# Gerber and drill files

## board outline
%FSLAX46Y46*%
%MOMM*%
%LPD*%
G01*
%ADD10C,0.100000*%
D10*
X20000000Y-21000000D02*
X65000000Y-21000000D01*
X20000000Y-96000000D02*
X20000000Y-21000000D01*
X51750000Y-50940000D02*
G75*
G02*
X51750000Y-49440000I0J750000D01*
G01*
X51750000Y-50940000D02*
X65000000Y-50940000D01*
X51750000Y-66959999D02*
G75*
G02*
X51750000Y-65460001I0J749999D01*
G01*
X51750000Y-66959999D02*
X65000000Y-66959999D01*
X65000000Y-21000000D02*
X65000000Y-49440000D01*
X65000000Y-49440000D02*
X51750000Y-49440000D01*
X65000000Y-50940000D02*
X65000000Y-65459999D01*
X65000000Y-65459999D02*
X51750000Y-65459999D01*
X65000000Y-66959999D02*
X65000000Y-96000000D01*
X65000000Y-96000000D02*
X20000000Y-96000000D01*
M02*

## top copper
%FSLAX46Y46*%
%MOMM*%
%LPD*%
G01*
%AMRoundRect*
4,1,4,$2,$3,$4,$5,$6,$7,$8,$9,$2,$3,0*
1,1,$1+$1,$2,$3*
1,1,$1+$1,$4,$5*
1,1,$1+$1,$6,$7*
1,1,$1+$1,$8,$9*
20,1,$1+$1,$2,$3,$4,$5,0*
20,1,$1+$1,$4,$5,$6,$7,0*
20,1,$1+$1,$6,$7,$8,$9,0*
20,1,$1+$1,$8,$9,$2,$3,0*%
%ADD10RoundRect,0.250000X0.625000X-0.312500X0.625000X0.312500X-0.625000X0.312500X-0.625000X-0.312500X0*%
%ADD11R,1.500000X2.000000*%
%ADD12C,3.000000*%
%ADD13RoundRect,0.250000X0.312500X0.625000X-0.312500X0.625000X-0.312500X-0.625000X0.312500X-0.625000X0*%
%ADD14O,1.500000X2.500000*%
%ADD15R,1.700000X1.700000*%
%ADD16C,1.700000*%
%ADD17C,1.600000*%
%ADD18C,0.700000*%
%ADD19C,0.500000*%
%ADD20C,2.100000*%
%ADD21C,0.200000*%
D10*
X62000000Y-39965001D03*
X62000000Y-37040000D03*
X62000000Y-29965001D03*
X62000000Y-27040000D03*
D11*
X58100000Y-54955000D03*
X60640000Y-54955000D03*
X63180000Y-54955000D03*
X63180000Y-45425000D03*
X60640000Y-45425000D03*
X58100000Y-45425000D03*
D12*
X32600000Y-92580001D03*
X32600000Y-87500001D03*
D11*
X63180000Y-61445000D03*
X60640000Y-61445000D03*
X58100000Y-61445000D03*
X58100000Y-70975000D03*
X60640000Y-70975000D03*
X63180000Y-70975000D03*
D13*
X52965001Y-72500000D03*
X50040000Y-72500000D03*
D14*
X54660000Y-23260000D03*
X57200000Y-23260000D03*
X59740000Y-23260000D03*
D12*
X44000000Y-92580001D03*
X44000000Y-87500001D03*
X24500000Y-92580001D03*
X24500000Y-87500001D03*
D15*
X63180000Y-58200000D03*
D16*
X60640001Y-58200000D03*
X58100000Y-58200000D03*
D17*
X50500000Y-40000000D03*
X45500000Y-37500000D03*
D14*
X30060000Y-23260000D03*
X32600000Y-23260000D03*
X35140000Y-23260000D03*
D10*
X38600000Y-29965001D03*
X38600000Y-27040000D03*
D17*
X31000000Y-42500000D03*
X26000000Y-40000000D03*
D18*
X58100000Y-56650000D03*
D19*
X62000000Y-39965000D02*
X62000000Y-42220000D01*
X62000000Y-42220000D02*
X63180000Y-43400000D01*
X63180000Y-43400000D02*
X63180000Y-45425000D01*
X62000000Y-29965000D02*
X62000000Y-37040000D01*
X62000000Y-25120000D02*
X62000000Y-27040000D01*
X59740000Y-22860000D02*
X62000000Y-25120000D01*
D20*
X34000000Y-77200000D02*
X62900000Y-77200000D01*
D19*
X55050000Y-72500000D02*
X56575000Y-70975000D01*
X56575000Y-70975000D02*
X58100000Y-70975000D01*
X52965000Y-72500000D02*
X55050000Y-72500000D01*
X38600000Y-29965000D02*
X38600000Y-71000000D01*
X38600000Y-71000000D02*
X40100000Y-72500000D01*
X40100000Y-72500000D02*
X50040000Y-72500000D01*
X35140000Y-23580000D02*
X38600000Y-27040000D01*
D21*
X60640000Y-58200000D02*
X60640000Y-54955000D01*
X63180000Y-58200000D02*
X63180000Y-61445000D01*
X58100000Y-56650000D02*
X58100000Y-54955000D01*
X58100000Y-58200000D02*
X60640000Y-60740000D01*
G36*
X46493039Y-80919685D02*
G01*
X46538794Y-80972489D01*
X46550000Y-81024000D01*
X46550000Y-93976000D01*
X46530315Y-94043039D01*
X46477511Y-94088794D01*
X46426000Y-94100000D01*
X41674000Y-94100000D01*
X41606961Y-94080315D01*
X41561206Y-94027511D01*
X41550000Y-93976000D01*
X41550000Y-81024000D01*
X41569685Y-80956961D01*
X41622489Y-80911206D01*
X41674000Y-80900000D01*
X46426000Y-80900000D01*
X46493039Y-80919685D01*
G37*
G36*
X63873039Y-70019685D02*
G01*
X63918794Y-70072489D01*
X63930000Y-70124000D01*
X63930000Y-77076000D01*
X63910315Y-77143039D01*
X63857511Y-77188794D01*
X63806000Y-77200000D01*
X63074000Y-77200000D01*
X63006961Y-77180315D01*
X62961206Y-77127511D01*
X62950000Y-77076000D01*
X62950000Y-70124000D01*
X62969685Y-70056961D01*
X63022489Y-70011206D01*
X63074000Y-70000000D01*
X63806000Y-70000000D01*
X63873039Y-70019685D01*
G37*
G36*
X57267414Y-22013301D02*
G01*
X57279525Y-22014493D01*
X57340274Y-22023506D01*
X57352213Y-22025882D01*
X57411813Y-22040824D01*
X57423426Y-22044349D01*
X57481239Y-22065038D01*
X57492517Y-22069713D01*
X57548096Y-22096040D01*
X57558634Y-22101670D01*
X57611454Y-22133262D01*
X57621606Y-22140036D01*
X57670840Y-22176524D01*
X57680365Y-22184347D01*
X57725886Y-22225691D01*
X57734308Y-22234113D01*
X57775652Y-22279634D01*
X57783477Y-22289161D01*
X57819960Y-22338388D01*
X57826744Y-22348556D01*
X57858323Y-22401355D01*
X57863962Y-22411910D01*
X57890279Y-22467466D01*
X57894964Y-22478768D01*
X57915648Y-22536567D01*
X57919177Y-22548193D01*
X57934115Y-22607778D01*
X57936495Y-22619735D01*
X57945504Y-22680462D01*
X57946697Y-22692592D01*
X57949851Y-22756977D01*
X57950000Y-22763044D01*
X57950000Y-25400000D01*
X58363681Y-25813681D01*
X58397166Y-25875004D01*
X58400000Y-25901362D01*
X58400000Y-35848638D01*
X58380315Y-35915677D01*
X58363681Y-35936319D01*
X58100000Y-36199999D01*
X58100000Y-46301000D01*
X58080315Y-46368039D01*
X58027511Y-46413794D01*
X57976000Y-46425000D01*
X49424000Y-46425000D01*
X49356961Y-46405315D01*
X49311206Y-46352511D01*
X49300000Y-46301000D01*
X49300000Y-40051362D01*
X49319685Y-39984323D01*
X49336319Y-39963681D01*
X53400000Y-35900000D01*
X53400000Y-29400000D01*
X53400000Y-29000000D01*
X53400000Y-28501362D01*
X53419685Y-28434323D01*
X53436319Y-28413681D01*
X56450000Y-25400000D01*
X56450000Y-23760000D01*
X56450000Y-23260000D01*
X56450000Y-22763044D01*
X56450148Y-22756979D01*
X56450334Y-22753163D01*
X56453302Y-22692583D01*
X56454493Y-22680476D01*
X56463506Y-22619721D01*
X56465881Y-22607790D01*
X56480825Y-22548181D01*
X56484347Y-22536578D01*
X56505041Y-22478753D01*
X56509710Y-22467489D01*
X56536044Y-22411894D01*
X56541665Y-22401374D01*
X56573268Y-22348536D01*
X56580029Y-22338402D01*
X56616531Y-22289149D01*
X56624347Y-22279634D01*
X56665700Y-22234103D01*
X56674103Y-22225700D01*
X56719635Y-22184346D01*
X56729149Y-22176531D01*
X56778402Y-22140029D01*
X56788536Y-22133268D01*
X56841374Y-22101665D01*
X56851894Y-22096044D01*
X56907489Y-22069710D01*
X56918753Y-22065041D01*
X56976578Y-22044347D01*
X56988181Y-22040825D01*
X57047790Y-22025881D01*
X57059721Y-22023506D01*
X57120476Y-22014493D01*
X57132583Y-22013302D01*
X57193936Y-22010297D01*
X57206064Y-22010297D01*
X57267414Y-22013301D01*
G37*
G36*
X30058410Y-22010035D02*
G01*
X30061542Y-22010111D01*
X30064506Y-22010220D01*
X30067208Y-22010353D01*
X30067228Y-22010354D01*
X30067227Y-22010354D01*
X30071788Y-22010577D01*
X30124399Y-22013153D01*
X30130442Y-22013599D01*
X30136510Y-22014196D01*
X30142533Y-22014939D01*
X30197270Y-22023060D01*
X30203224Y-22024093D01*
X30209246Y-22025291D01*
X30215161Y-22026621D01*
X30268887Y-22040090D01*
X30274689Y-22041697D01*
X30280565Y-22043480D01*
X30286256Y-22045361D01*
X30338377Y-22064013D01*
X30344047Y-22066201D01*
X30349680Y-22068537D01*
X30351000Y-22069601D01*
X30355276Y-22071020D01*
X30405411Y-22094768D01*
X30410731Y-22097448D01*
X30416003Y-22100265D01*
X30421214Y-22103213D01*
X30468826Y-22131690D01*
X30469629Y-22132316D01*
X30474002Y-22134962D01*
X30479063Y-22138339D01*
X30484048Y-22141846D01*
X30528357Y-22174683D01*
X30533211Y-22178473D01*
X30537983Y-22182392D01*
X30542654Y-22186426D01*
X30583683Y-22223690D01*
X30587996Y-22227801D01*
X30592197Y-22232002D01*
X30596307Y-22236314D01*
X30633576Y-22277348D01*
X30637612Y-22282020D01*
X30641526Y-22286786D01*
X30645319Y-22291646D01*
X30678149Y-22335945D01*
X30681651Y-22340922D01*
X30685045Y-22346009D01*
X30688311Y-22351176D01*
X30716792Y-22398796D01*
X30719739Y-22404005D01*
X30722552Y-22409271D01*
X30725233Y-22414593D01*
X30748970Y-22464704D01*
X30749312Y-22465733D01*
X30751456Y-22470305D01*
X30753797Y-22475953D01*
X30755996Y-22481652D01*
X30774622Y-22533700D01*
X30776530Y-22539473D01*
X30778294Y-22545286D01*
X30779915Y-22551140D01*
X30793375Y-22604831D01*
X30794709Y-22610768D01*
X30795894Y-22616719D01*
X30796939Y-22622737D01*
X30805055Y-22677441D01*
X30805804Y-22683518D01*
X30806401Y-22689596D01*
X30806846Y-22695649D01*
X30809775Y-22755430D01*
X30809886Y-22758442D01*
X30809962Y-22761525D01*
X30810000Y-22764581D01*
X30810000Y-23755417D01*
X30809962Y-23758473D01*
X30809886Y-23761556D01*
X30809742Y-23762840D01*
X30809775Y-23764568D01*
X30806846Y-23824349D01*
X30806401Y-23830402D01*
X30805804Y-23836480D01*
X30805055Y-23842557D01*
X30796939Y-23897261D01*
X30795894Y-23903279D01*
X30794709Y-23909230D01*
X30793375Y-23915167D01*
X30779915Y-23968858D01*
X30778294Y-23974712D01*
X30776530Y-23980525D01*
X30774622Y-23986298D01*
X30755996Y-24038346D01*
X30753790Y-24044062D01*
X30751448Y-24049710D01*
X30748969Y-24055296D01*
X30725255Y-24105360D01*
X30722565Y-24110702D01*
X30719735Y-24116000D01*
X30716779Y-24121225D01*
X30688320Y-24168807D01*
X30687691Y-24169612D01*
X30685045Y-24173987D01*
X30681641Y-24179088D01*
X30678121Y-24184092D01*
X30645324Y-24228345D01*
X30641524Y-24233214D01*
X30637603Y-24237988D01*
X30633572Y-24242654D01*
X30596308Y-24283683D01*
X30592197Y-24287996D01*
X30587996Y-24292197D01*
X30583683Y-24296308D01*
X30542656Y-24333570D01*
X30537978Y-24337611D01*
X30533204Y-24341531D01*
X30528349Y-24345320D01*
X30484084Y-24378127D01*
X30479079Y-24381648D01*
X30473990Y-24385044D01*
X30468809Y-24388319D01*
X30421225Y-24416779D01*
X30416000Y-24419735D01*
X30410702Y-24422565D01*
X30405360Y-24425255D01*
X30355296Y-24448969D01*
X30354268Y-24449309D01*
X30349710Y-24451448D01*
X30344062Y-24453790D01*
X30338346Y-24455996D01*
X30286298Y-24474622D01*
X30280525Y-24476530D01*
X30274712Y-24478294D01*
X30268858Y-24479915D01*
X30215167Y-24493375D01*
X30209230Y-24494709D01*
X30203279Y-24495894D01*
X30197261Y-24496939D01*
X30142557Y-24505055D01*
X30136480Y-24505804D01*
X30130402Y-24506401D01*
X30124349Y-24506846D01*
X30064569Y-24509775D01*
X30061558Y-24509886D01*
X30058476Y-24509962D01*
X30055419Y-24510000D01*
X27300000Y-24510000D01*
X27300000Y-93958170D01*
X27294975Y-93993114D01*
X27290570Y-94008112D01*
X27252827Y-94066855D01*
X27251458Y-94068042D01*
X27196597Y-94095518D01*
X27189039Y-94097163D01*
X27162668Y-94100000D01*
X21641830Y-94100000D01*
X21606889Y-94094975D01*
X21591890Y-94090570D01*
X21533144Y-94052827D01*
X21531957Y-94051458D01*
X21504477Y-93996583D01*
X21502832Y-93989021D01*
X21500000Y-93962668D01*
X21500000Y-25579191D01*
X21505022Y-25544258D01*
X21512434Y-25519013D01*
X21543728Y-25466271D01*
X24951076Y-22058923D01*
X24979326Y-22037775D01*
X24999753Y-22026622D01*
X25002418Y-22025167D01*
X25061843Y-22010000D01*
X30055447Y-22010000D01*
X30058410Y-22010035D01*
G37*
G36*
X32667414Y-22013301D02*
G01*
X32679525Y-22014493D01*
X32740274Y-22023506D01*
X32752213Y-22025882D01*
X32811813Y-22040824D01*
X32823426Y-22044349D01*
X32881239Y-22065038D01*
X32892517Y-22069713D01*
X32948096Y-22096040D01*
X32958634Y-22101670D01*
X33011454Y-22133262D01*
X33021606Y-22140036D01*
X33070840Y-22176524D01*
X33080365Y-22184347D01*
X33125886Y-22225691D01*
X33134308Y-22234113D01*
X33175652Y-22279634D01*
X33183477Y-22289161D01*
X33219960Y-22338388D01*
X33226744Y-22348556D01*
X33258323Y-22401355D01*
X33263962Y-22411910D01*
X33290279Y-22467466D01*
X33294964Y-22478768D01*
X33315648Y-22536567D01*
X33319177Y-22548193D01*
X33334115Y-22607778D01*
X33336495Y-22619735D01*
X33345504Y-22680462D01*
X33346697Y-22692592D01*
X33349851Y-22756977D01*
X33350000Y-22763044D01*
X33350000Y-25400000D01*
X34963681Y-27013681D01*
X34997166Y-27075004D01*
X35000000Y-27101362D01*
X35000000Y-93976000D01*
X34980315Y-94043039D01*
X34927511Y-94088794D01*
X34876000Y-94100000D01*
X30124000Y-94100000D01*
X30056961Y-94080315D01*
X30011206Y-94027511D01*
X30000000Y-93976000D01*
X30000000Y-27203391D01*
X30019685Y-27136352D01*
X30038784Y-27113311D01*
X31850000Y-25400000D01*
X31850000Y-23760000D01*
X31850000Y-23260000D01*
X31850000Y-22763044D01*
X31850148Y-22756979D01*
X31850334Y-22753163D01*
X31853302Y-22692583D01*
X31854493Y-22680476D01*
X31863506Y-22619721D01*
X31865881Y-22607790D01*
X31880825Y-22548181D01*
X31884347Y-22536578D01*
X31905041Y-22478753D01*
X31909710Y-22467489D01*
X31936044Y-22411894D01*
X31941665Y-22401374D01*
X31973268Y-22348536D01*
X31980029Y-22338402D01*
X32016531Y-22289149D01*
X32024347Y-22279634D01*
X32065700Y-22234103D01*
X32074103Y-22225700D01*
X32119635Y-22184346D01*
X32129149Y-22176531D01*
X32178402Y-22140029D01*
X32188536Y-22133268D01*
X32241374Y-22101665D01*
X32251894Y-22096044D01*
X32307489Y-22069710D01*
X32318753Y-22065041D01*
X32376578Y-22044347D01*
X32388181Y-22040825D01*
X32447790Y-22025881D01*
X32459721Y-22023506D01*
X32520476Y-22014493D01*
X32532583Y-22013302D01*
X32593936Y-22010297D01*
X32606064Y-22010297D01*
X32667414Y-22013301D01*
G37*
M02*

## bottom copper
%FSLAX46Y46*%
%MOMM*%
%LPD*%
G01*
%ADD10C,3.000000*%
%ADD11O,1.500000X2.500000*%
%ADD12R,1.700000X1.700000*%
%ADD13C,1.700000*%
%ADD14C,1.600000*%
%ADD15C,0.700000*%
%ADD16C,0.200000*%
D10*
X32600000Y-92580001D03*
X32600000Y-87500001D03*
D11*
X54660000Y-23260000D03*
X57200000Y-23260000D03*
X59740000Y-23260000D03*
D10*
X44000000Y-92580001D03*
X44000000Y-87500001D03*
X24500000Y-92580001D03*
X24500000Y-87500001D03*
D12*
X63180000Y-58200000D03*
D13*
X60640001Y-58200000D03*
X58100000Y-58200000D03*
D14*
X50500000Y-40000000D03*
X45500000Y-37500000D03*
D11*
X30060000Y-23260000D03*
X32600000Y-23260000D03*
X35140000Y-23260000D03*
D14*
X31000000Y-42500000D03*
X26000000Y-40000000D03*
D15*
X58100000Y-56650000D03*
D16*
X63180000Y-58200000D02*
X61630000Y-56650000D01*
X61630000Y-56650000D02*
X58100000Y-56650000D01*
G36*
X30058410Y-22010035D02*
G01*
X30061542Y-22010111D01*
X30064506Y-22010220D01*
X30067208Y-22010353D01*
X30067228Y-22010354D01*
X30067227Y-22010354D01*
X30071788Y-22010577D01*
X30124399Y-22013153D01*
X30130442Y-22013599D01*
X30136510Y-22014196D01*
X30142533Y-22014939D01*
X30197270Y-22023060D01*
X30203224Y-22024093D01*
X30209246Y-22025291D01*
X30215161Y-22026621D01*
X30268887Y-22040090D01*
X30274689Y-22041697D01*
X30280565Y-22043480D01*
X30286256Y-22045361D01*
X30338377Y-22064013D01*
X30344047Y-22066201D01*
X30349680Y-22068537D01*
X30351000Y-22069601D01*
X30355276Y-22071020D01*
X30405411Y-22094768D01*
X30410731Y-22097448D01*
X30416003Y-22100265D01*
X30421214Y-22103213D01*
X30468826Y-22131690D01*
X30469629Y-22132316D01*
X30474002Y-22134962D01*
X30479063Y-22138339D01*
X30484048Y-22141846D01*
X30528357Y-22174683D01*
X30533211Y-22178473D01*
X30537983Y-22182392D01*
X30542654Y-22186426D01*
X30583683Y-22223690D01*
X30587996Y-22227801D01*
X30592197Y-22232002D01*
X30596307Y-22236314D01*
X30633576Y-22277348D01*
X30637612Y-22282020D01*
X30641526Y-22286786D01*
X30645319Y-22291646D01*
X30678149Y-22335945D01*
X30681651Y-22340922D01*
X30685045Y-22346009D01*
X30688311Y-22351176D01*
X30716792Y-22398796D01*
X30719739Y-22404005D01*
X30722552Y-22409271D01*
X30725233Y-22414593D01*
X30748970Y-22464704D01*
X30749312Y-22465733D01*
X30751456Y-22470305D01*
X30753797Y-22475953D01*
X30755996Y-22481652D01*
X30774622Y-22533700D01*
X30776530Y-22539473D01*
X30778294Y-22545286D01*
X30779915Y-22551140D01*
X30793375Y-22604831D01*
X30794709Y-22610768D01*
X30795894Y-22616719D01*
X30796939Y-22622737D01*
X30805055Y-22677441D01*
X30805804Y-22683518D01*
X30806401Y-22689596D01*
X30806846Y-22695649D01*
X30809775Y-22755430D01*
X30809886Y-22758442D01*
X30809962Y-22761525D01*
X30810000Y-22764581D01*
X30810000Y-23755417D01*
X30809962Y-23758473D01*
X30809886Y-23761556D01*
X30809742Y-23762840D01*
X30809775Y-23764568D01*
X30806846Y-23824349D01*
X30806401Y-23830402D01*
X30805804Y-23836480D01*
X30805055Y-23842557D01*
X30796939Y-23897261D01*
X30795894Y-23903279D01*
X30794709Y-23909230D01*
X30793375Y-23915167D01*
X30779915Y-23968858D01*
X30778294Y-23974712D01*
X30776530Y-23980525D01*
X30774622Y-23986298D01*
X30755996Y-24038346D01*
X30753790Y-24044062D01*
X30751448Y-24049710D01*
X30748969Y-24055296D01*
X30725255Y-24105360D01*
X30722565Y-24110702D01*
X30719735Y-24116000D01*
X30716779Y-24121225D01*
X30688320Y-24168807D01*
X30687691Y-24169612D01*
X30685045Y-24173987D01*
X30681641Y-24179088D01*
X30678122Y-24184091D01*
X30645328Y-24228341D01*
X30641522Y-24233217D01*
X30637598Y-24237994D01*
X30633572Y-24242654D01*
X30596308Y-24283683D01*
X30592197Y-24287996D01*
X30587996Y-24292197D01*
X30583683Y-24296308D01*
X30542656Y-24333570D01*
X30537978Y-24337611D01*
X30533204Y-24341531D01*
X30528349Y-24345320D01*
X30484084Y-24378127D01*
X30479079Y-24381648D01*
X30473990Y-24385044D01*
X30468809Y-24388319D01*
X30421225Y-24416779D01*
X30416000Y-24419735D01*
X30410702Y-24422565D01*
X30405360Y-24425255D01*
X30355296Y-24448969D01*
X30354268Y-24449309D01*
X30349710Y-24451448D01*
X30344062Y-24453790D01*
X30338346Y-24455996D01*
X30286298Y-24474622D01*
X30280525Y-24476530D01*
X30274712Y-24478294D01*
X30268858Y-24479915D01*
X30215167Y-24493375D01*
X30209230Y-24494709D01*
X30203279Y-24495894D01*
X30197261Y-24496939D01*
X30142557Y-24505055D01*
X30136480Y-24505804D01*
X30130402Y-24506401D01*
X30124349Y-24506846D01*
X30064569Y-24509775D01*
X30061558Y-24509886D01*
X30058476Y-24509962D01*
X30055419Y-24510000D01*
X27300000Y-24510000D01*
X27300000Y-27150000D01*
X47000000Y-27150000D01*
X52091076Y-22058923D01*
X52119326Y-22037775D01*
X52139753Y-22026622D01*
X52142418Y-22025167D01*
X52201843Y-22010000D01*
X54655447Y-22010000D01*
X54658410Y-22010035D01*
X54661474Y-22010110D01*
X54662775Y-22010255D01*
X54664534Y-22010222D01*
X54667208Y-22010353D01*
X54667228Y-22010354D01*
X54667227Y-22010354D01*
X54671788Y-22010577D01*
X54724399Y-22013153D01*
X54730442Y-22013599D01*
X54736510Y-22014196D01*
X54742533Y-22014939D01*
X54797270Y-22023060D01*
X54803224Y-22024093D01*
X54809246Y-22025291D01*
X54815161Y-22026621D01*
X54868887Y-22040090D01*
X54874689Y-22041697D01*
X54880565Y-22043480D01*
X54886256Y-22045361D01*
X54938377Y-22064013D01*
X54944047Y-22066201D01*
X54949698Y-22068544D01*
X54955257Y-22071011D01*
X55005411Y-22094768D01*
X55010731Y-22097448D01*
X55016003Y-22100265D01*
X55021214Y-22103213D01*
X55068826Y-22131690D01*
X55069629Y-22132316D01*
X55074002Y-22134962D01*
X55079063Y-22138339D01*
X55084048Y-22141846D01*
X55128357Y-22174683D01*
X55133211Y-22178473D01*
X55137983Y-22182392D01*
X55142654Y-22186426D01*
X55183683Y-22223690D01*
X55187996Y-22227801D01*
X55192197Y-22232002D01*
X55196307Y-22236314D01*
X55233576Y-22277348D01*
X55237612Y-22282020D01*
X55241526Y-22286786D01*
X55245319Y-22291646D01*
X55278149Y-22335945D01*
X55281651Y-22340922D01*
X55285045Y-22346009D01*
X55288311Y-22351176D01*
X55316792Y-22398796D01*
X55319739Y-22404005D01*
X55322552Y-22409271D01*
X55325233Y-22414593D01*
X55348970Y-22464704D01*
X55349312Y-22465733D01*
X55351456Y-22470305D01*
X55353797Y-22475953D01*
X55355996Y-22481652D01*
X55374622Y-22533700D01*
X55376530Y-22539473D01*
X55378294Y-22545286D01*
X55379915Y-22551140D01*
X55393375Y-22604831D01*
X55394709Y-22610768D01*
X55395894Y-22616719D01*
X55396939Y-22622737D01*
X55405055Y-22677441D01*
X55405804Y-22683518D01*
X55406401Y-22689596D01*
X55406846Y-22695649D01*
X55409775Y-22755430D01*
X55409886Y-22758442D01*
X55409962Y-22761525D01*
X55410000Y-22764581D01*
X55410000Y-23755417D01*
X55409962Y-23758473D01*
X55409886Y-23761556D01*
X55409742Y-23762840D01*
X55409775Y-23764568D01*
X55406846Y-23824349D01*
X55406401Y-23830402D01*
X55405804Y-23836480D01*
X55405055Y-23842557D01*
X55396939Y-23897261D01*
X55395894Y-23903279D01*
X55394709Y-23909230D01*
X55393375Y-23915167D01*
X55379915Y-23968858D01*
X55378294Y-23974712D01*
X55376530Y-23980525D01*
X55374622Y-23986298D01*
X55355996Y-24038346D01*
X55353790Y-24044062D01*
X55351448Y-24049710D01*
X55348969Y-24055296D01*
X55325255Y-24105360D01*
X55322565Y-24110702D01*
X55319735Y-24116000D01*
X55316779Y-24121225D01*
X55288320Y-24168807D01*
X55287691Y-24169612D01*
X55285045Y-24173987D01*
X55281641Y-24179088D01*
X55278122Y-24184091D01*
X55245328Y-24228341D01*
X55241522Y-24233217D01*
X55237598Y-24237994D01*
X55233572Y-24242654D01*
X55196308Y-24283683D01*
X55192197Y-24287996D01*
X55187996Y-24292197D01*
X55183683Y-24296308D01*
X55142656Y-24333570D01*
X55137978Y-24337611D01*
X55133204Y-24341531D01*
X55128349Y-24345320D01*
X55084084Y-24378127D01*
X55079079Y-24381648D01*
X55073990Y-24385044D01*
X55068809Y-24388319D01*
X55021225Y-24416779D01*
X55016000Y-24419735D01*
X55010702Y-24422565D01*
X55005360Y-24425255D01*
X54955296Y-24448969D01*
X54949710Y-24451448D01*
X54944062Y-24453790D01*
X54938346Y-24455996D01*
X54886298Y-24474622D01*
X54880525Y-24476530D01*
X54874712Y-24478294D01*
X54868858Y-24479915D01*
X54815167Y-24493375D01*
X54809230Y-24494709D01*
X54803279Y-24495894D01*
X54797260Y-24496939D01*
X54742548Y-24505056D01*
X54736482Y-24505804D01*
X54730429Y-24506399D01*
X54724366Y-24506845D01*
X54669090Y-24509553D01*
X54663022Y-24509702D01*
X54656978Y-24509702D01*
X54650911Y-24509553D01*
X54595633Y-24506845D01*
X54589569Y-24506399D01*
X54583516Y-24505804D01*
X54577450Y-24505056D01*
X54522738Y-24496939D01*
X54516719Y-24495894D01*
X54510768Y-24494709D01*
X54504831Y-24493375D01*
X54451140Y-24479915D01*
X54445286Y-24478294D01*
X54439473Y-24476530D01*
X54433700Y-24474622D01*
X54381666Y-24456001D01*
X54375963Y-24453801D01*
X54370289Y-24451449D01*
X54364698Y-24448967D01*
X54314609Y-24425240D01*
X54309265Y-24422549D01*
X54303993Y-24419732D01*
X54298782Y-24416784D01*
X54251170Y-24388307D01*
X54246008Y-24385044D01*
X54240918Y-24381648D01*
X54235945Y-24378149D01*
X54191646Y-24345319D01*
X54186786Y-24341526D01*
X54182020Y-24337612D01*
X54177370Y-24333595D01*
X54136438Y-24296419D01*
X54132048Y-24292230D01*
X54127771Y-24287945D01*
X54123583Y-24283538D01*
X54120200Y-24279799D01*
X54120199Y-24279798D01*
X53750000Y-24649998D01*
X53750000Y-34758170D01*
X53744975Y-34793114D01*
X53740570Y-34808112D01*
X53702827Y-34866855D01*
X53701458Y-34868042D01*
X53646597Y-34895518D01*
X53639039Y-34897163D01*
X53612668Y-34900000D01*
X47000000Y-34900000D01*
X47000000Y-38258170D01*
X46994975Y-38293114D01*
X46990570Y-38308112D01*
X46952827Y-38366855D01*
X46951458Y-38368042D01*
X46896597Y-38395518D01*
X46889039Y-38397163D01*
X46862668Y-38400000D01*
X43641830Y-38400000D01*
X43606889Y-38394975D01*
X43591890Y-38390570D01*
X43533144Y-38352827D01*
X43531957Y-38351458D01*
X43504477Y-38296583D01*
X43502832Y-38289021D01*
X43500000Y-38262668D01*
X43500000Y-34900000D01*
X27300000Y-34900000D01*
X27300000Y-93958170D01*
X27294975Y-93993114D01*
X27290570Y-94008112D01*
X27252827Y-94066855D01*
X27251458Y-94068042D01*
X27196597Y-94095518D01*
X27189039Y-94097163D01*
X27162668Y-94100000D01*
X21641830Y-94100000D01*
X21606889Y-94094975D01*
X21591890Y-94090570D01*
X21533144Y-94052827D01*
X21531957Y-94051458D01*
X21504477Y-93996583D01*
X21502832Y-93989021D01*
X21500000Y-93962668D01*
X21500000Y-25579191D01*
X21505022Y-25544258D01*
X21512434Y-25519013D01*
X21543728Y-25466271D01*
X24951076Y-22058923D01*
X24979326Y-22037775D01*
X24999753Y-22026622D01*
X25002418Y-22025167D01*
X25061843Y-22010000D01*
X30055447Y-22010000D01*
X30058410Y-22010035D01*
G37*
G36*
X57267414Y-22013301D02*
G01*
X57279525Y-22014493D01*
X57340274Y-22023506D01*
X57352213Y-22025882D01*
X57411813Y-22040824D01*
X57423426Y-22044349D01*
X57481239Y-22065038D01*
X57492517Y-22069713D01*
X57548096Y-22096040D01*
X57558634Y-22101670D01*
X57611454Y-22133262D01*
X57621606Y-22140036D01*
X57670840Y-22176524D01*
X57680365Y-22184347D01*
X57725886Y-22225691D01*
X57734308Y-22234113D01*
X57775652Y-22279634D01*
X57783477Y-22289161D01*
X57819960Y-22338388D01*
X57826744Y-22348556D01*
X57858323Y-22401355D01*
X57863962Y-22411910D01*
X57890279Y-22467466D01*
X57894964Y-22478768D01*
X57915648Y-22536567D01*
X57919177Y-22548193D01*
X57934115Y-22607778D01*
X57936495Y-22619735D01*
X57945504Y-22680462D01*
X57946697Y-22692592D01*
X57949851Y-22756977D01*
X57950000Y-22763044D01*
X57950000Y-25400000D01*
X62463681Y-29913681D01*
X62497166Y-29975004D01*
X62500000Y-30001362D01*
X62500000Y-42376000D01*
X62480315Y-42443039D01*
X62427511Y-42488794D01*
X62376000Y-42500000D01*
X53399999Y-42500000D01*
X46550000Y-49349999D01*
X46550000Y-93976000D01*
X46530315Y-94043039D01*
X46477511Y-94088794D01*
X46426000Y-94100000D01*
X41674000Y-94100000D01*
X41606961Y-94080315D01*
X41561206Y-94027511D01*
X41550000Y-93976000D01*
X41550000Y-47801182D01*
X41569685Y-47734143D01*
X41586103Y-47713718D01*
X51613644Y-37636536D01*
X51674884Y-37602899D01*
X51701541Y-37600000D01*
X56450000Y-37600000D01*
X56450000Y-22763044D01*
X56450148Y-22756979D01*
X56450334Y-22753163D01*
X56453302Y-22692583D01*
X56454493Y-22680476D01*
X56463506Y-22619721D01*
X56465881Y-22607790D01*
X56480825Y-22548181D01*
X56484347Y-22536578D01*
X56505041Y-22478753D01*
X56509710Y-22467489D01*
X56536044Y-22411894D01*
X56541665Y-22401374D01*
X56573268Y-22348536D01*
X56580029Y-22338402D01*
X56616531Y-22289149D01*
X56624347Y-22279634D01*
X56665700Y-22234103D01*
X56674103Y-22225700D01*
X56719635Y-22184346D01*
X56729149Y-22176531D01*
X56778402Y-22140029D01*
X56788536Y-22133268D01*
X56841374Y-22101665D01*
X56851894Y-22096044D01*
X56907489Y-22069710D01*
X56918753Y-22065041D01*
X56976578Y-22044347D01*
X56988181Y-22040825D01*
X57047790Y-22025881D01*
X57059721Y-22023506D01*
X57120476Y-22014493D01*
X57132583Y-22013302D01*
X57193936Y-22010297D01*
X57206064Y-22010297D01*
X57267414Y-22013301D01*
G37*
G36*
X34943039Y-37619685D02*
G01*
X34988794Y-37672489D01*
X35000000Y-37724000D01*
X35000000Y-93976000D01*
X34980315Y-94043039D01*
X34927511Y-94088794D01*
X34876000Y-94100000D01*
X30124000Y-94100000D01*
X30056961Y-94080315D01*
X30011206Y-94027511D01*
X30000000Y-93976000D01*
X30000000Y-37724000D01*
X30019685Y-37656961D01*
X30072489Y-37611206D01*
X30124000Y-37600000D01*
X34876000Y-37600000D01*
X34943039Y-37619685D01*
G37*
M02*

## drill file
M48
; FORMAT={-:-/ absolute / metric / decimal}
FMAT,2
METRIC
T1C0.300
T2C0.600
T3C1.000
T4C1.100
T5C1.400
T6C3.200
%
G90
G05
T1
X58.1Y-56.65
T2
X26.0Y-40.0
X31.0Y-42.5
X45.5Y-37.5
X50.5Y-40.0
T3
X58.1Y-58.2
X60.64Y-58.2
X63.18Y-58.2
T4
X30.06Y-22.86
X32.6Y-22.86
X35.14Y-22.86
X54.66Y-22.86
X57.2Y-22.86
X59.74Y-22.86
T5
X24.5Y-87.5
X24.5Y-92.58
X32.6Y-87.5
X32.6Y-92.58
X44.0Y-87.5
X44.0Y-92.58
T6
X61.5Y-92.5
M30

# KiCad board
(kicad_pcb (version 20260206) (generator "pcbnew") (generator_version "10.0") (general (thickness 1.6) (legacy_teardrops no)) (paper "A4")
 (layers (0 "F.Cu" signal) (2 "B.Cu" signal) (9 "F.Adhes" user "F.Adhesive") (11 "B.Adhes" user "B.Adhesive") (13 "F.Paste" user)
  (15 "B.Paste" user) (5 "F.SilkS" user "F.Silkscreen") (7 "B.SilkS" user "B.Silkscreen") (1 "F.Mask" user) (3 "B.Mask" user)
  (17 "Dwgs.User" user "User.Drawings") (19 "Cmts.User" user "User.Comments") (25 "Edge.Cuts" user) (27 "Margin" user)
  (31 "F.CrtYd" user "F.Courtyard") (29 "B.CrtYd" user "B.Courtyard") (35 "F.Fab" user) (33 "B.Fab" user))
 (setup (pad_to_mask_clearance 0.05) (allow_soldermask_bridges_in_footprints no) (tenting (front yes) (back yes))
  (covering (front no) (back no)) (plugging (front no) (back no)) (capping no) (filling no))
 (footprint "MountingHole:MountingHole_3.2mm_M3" (layer "F.Cu") (at 61.5 92.5)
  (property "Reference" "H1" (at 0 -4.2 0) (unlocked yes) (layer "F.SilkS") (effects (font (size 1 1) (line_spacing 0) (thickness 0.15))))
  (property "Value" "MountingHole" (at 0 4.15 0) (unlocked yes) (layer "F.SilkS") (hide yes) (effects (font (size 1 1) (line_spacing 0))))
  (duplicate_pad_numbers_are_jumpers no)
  (pad "" np_thru_hole circle (at 0 0) (size 3.2 3.2) (drill 3.2) (layers "*.Cu" "*.Mask")))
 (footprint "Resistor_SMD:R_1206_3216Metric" (layer "F.Cu") (at 62 38.502501 90)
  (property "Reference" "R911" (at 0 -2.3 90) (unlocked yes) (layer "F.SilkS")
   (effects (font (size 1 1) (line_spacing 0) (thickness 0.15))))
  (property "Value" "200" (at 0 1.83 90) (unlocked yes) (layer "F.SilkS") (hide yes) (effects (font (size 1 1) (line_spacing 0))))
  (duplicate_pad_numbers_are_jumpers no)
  (pad "1" smd roundrect (at -1.4625 0 90) (size 1.125 1.75) (layers "F.Cu" "F.Mask" "F.Paste") (roundrect_rratio 0.222222)
   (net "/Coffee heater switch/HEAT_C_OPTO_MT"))
  (pad "2" smd roundrect (at 1.462501 0 90) (size 1.125 1.75) (layers "F.Cu" "F.Mask" "F.Paste") (roundrect_rratio 0.222222)
   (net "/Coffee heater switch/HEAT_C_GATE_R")))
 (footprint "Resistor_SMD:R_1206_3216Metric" (layer "F.Cu") (at 62 28.502501 90)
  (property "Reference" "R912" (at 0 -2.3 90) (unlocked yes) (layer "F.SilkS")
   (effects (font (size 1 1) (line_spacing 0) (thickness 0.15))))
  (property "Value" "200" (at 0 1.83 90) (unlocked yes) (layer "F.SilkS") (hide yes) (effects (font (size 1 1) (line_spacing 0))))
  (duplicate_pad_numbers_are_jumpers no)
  (pad "1" smd roundrect (at -1.4625 0 90) (size 1.125 1.75) (layers "F.Cu" "F.Mask" "F.Paste") (roundrect_rratio 0.222222)
   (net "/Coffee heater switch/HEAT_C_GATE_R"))
  (pad "2" smd roundrect (at 1.462501 0 90) (size 1.125 1.75) (layers "F.Cu" "F.Mask" "F.Paste") (roundrect_rratio 0.222222)
   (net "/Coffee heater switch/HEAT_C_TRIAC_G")))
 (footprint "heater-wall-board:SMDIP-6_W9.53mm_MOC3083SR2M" (layer "F.Cu") (at 60.64 50.19 90)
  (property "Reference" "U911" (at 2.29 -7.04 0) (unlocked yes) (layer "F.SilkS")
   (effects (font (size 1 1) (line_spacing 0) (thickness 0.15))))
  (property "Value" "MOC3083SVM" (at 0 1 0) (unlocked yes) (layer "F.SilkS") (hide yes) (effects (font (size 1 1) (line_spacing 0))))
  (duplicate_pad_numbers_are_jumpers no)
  (pad "1" smd rect (at -4.765 -2.54 90) (size 2 1.5) (layers "F.Cu" "F.Mask" "F.Paste") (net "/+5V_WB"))
  (pad "2" smd rect (at -4.765 0 90) (size 2 1.5) (layers "F.Cu" "F.Mask" "F.Paste") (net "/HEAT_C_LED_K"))
  (pad "3" smd rect (at -4.765 2.54 90) (size 2 1.5) (layers "F.Cu" "F.Mask" "F.Paste") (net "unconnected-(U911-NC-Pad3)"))
  (pad "4" smd rect (at 4.765 2.54 90) (size 2 1.5) (layers "F.Cu" "F.Mask" "F.Paste") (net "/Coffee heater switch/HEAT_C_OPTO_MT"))
  (pad "5" smd rect (at 4.765 0 90) (size 2 1.5) (layers "F.Cu" "F.Mask" "F.Paste") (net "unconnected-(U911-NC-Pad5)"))
  (pad "6" smd rect (at 4.765 -2.54 90) (size 2 1.5) (layers "F.Cu" "F.Mask" "F.Paste") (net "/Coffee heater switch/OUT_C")))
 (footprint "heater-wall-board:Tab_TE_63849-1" (layer "F.Cu") (at 32.6 90.04 90)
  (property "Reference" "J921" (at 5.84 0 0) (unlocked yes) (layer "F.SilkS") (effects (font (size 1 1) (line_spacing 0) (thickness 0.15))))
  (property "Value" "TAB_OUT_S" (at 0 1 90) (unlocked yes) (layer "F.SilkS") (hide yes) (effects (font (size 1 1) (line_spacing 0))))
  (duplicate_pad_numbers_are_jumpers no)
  (pad "1" thru_hole circle (at -2.540001 0 90) (size 3 3) (drill 1.4) (layers "*.Cu" "*.Mask") (remove_unused_layers no)
   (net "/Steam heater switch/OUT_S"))
  (pad "1" thru_hole circle (at 2.539999 0 90) (size 3 3) (drill 1.4) (layers "*.Cu" "*.Mask") (remove_unused_layers no)
   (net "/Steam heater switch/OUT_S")))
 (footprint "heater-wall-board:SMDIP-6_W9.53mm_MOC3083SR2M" (layer "F.Cu") (at 60.64 66.21 -90)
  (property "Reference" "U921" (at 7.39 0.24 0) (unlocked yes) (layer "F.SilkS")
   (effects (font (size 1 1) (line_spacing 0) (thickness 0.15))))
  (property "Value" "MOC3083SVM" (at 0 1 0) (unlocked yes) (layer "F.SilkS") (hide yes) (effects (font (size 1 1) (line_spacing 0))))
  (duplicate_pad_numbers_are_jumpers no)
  (pad "1" smd rect (at -4.765 -2.54 270) (size 2 1.5) (layers "F.Cu" "F.Mask" "F.Paste") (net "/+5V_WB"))
  (pad "2" smd rect (at -4.765 0 270) (size 2 1.5) (layers "F.Cu" "F.Mask" "F.Paste") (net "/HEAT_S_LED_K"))
  (pad "3" smd rect (at -4.765 2.54 270) (size 2 1.5) (layers "F.Cu" "F.Mask" "F.Paste") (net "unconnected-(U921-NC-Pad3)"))
  (pad "4" smd rect (at 4.765 2.54 270) (size 2 1.5) (layers "F.Cu" "F.Mask" "F.Paste") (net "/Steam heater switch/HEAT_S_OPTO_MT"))
  (pad "5" smd rect (at 4.765 0 270) (size 2 1.5) (layers "F.Cu" "F.Mask" "F.Paste") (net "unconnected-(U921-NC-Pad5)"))
  (pad "6" smd rect (at 4.765 -2.54 270) (size 2 1.5) (layers "F.Cu" "F.Mask" "F.Paste") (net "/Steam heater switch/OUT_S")))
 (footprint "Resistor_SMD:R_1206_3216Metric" (layer "F.Cu") (at 51.502501 72.5 180)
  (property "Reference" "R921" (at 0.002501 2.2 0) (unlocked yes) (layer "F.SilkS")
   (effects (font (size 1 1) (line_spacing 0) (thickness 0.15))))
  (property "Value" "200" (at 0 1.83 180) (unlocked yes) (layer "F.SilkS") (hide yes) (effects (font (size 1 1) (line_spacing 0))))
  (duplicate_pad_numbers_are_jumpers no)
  (pad "1" smd roundrect (at -1.4625 0 180) (size 1.125 1.75) (layers "F.Cu" "F.Mask" "F.Paste") (roundrect_rratio 0.222222)
   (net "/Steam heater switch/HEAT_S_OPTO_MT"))
  (pad "2" smd roundrect (at 1.462501 0 180) (size 1.125 1.75) (layers "F.Cu" "F.Mask" "F.Paste") (roundrect_rratio 0.222222)
   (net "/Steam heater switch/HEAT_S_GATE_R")))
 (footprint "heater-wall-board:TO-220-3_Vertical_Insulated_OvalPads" (layer "F.Cu") (at 54.66 22.86)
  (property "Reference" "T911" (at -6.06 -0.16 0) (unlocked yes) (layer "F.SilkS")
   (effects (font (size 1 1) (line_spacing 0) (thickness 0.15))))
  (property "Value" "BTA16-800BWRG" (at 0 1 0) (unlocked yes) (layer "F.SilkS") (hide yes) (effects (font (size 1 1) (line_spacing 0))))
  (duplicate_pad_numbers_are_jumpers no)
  (pad "1" thru_hole oval (at 0 0) (size 1.5 2.5) (drill 1.1 (offset 0 0.4)) (layers "*.Cu" "*.Mask") (remove_unused_layers no) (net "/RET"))
  (pad "2" thru_hole oval (at 2.54 0) (size 1.5 2.5) (drill 1.1 (offset 0 0.4)) (layers "*.Cu" "*.Mask") (remove_unused_layers no)
   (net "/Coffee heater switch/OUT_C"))
  (pad "3" thru_hole oval (at 5.08 0) (size 1.5 2.5) (drill 1.1 (offset 0 0.4)) (layers "*.Cu" "*.Mask") (remove_unused_layers no)
   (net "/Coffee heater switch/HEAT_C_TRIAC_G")))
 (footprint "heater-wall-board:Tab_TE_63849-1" (layer "F.Cu") (at 44 90.04 90)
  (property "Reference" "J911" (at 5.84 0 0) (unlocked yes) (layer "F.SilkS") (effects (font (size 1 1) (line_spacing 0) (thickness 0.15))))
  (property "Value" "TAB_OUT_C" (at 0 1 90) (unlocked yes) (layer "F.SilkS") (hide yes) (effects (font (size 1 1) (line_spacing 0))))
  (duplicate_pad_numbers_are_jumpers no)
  (pad "1" thru_hole circle (at -2.540001 0 90) (size 3 3) (drill 1.4) (layers "*.Cu" "*.Mask") (remove_unused_layers no)
   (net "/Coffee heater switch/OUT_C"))
  (pad "1" thru_hole circle (at 2.539999 0 90) (size 3 3) (drill 1.4) (layers "*.Cu" "*.Mask") (remove_unused_layers no)
   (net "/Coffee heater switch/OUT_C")))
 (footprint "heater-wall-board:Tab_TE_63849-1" (layer "F.Cu") (at 24.5 90.04 90)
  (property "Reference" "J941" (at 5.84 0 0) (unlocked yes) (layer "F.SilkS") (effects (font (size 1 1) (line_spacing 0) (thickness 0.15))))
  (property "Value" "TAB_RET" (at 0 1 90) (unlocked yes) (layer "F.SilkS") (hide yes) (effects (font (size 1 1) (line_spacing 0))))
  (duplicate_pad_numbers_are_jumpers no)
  (pad "1" thru_hole circle (at -2.540001 0 90) (size 3 3) (drill 1.4) (layers "*.Cu" "*.Mask") (remove_unused_layers no) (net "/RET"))
  (pad "1" thru_hole circle (at 2.539999 0 90) (size 3 3) (drill 1.4) (layers "*.Cu" "*.Mask") (remove_unused_layers no) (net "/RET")))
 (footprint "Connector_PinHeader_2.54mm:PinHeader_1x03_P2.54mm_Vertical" (layer "F.Cu") (at 63.18 58.2 -90)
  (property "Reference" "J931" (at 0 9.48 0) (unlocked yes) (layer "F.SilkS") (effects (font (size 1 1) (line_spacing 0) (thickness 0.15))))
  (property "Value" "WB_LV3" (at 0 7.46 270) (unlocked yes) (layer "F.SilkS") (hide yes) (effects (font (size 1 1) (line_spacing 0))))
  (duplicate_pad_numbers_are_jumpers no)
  (pad "1" thru_hole rect (at 0 0 270) (size 1.7 1.7) (drill 1) (layers "*.Cu" "*.Mask") (remove_unused_layers no) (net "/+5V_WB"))
  (pad "2" thru_hole circle (at 0 2.539999 270) (size 1.7 1.7) (drill 1) (layers "*.Cu" "*.Mask") (remove_unused_layers no)
   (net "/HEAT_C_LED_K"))
  (pad "3" thru_hole circle (at 0 5.08 270) (size 1.7 1.7) (drill 1) (layers "*.Cu" "*.Mask") (remove_unused_layers no)
   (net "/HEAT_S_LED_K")))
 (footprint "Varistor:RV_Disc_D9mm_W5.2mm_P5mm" (layer "F.Cu") (at 50.5 40 180)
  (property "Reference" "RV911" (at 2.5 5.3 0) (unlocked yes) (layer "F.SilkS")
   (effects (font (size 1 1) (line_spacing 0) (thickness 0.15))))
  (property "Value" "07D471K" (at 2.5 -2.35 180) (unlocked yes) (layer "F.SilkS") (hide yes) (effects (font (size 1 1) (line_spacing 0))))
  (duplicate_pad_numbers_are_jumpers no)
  (pad "1" thru_hole circle (at 0 0 180) (size 1.6 1.6) (drill 0.6) (layers "*.Cu" "*.Mask") (remove_unused_layers no)
   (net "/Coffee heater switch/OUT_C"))
  (pad "2" thru_hole circle (at 5 2.5 180) (size 1.6 1.6) (drill 0.6) (layers "*.Cu" "*.Mask") (remove_unused_layers no) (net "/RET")))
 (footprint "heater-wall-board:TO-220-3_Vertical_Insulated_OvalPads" (layer "F.Cu") (at 30.06 22.86)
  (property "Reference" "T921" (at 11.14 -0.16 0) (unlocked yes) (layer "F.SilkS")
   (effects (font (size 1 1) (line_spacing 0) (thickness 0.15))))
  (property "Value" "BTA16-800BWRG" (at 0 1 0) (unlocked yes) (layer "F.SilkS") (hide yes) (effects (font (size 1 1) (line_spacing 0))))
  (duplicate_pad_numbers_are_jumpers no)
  (pad "1" thru_hole oval (at 0 0) (size 1.5 2.5) (drill 1.1 (offset 0 0.4)) (layers "*.Cu" "*.Mask") (remove_unused_layers no) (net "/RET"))
  (pad "2" thru_hole oval (at 2.54 0) (size 1.5 2.5) (drill 1.1 (offset 0 0.4)) (layers "*.Cu" "*.Mask") (remove_unused_layers no)
   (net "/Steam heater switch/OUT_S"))
  (pad "3" thru_hole oval (at 5.08 0) (size 1.5 2.5) (drill 1.1 (offset 0 0.4)) (layers "*.Cu" "*.Mask") (remove_unused_layers no)
   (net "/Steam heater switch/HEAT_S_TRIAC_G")))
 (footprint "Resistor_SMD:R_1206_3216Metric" (layer "F.Cu") (at 38.6 28.502501 90)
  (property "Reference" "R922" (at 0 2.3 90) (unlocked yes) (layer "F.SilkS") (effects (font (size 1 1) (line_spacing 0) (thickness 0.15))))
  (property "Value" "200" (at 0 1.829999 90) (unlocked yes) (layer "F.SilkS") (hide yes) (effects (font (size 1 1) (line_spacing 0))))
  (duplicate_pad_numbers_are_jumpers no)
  (pad "1" smd roundrect (at -1.4625 0 90) (size 1.125 1.75) (layers "F.Cu" "F.Mask" "F.Paste") (roundrect_rratio 0.222222)
   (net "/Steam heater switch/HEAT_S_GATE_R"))
  (pad "2" smd roundrect (at 1.462501 0 90) (size 1.125 1.75) (layers "F.Cu" "F.Mask" "F.Paste") (roundrect_rratio 0.222222)
   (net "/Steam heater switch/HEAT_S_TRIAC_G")))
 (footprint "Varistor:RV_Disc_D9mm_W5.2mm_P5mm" (layer "F.Cu") (at 31 42.5 180)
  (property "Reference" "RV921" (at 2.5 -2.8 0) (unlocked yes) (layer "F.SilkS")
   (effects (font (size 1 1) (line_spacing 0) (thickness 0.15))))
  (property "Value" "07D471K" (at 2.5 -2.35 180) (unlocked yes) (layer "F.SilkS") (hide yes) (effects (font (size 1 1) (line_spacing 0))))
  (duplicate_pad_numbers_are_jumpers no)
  (pad "1" thru_hole circle (at 0 0 180) (size 1.6 1.6) (drill 0.6) (layers "*.Cu" "*.Mask") (remove_unused_layers no)
   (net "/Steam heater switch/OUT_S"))
  (pad "2" thru_hole circle (at 5 2.5 180) (size 1.6 1.6) (drill 0.6) (layers "*.Cu" "*.Mask") (remove_unused_layers no) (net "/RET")))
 (gr_line (start 20 21) (end 65 21) (stroke (width 0.1) (type default)) (layer "Edge.Cuts"))
 (gr_line (start 20 96) (end 20 21) (stroke (width 0.1) (type default)) (layer "Edge.Cuts"))
 (gr_arc (start 51.75 50.94) (mid 51 50.19) (end 51.75 49.44) (stroke (width 0.1) (type default)) (layer "Edge.Cuts"))
 (gr_line (start 51.75 50.94) (end 65 50.94) (stroke (width 0.1) (type default)) (layer "Edge.Cuts"))
 (gr_arc (start 51.75 66.959999) (mid 51.000001 66.21) (end 51.75 65.459999) (stroke (width 0.1) (type default)) (layer "Edge.Cuts"))
 (gr_line (start 51.75 66.959999) (end 65 66.959999) (stroke (width 0.1) (type default)) (layer "Edge.Cuts"))
 (gr_line (start 65 21) (end 65 49.44) (stroke (width 0.1) (type default)) (layer "Edge.Cuts"))
 (gr_line (start 65 49.44) (end 51.75 49.44) (stroke (width 0.1) (type default)) (layer "Edge.Cuts"))
 (gr_line (start 65 50.94) (end 65 65.459999) (stroke (width 0.1) (type default)) (layer "Edge.Cuts"))
 (gr_line (start 65 65.459999) (end 51.75 65.459999) (stroke (width 0.1) (type default)) (layer "Edge.Cuts"))
 (gr_line (start 65 66.959999) (end 65 96) (stroke (width 0.1) (type default)) (layer "Edge.Cuts"))
 (gr_line (start 65 96) (end 20 96) (stroke (width 0.1) (type default)) (layer "Edge.Cuts"))
 (segment (start 62 39.965) (end 62 42.22) (width 0.5) (locked yes) (layer "F.Cu") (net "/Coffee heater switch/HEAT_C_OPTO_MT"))
 (segment (start 62 42.22) (end 63.18 43.4) (width 0.5) (locked yes) (layer "F.Cu") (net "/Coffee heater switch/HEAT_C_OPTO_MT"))
 (segment (start 63.18 43.4) (end 63.18 45.425) (width 0.5) (locked yes) (layer "F.Cu") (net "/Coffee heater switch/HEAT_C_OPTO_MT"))
 (segment (start 62 29.965) (end 62 37.04) (width 0.5) (locked yes) (layer "F.Cu") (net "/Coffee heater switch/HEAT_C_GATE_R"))
 (segment (start 62 25.12) (end 62 27.04) (width 0.5) (locked yes) (layer "F.Cu") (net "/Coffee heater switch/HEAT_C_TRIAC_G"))
 (segment (start 59.74 22.86) (end 62 25.12) (width 0.5) (locked yes) (layer "F.Cu") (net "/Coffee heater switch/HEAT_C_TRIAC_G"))
 (segment (start 34 77.2) (end 62.9 77.2) (width 2.1) (locked yes) (layer "F.Cu") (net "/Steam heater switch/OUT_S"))
 (segment (start 55.05 72.5) (end 56.575 70.975) (width 0.5) (locked yes) (layer "F.Cu") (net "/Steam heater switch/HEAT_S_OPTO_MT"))
 (segment (start 56.575 70.975) (end 58.1 70.975) (width 0.5) (locked yes) (layer "F.Cu") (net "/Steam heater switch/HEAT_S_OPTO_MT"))
 (segment (start 52.965 72.5) (end 55.05 72.5) (width 0.5) (locked yes) (layer "F.Cu") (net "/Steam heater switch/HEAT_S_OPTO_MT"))
 (segment (start 38.6 29.965) (end 38.6 71) (width 0.5) (locked yes) (layer "F.Cu") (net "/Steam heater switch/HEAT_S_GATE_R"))
 (segment (start 38.6 71) (end 40.1 72.5) (width 0.5) (locked yes) (layer "F.Cu") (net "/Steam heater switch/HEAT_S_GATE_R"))
 (segment (start 40.1 72.5) (end 50.04 72.5) (width 0.5) (locked yes) (layer "F.Cu") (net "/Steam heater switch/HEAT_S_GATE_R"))
 (segment (start 35.14 23.58) (end 38.6 27.04) (width 0.5) (locked yes) (layer "F.Cu") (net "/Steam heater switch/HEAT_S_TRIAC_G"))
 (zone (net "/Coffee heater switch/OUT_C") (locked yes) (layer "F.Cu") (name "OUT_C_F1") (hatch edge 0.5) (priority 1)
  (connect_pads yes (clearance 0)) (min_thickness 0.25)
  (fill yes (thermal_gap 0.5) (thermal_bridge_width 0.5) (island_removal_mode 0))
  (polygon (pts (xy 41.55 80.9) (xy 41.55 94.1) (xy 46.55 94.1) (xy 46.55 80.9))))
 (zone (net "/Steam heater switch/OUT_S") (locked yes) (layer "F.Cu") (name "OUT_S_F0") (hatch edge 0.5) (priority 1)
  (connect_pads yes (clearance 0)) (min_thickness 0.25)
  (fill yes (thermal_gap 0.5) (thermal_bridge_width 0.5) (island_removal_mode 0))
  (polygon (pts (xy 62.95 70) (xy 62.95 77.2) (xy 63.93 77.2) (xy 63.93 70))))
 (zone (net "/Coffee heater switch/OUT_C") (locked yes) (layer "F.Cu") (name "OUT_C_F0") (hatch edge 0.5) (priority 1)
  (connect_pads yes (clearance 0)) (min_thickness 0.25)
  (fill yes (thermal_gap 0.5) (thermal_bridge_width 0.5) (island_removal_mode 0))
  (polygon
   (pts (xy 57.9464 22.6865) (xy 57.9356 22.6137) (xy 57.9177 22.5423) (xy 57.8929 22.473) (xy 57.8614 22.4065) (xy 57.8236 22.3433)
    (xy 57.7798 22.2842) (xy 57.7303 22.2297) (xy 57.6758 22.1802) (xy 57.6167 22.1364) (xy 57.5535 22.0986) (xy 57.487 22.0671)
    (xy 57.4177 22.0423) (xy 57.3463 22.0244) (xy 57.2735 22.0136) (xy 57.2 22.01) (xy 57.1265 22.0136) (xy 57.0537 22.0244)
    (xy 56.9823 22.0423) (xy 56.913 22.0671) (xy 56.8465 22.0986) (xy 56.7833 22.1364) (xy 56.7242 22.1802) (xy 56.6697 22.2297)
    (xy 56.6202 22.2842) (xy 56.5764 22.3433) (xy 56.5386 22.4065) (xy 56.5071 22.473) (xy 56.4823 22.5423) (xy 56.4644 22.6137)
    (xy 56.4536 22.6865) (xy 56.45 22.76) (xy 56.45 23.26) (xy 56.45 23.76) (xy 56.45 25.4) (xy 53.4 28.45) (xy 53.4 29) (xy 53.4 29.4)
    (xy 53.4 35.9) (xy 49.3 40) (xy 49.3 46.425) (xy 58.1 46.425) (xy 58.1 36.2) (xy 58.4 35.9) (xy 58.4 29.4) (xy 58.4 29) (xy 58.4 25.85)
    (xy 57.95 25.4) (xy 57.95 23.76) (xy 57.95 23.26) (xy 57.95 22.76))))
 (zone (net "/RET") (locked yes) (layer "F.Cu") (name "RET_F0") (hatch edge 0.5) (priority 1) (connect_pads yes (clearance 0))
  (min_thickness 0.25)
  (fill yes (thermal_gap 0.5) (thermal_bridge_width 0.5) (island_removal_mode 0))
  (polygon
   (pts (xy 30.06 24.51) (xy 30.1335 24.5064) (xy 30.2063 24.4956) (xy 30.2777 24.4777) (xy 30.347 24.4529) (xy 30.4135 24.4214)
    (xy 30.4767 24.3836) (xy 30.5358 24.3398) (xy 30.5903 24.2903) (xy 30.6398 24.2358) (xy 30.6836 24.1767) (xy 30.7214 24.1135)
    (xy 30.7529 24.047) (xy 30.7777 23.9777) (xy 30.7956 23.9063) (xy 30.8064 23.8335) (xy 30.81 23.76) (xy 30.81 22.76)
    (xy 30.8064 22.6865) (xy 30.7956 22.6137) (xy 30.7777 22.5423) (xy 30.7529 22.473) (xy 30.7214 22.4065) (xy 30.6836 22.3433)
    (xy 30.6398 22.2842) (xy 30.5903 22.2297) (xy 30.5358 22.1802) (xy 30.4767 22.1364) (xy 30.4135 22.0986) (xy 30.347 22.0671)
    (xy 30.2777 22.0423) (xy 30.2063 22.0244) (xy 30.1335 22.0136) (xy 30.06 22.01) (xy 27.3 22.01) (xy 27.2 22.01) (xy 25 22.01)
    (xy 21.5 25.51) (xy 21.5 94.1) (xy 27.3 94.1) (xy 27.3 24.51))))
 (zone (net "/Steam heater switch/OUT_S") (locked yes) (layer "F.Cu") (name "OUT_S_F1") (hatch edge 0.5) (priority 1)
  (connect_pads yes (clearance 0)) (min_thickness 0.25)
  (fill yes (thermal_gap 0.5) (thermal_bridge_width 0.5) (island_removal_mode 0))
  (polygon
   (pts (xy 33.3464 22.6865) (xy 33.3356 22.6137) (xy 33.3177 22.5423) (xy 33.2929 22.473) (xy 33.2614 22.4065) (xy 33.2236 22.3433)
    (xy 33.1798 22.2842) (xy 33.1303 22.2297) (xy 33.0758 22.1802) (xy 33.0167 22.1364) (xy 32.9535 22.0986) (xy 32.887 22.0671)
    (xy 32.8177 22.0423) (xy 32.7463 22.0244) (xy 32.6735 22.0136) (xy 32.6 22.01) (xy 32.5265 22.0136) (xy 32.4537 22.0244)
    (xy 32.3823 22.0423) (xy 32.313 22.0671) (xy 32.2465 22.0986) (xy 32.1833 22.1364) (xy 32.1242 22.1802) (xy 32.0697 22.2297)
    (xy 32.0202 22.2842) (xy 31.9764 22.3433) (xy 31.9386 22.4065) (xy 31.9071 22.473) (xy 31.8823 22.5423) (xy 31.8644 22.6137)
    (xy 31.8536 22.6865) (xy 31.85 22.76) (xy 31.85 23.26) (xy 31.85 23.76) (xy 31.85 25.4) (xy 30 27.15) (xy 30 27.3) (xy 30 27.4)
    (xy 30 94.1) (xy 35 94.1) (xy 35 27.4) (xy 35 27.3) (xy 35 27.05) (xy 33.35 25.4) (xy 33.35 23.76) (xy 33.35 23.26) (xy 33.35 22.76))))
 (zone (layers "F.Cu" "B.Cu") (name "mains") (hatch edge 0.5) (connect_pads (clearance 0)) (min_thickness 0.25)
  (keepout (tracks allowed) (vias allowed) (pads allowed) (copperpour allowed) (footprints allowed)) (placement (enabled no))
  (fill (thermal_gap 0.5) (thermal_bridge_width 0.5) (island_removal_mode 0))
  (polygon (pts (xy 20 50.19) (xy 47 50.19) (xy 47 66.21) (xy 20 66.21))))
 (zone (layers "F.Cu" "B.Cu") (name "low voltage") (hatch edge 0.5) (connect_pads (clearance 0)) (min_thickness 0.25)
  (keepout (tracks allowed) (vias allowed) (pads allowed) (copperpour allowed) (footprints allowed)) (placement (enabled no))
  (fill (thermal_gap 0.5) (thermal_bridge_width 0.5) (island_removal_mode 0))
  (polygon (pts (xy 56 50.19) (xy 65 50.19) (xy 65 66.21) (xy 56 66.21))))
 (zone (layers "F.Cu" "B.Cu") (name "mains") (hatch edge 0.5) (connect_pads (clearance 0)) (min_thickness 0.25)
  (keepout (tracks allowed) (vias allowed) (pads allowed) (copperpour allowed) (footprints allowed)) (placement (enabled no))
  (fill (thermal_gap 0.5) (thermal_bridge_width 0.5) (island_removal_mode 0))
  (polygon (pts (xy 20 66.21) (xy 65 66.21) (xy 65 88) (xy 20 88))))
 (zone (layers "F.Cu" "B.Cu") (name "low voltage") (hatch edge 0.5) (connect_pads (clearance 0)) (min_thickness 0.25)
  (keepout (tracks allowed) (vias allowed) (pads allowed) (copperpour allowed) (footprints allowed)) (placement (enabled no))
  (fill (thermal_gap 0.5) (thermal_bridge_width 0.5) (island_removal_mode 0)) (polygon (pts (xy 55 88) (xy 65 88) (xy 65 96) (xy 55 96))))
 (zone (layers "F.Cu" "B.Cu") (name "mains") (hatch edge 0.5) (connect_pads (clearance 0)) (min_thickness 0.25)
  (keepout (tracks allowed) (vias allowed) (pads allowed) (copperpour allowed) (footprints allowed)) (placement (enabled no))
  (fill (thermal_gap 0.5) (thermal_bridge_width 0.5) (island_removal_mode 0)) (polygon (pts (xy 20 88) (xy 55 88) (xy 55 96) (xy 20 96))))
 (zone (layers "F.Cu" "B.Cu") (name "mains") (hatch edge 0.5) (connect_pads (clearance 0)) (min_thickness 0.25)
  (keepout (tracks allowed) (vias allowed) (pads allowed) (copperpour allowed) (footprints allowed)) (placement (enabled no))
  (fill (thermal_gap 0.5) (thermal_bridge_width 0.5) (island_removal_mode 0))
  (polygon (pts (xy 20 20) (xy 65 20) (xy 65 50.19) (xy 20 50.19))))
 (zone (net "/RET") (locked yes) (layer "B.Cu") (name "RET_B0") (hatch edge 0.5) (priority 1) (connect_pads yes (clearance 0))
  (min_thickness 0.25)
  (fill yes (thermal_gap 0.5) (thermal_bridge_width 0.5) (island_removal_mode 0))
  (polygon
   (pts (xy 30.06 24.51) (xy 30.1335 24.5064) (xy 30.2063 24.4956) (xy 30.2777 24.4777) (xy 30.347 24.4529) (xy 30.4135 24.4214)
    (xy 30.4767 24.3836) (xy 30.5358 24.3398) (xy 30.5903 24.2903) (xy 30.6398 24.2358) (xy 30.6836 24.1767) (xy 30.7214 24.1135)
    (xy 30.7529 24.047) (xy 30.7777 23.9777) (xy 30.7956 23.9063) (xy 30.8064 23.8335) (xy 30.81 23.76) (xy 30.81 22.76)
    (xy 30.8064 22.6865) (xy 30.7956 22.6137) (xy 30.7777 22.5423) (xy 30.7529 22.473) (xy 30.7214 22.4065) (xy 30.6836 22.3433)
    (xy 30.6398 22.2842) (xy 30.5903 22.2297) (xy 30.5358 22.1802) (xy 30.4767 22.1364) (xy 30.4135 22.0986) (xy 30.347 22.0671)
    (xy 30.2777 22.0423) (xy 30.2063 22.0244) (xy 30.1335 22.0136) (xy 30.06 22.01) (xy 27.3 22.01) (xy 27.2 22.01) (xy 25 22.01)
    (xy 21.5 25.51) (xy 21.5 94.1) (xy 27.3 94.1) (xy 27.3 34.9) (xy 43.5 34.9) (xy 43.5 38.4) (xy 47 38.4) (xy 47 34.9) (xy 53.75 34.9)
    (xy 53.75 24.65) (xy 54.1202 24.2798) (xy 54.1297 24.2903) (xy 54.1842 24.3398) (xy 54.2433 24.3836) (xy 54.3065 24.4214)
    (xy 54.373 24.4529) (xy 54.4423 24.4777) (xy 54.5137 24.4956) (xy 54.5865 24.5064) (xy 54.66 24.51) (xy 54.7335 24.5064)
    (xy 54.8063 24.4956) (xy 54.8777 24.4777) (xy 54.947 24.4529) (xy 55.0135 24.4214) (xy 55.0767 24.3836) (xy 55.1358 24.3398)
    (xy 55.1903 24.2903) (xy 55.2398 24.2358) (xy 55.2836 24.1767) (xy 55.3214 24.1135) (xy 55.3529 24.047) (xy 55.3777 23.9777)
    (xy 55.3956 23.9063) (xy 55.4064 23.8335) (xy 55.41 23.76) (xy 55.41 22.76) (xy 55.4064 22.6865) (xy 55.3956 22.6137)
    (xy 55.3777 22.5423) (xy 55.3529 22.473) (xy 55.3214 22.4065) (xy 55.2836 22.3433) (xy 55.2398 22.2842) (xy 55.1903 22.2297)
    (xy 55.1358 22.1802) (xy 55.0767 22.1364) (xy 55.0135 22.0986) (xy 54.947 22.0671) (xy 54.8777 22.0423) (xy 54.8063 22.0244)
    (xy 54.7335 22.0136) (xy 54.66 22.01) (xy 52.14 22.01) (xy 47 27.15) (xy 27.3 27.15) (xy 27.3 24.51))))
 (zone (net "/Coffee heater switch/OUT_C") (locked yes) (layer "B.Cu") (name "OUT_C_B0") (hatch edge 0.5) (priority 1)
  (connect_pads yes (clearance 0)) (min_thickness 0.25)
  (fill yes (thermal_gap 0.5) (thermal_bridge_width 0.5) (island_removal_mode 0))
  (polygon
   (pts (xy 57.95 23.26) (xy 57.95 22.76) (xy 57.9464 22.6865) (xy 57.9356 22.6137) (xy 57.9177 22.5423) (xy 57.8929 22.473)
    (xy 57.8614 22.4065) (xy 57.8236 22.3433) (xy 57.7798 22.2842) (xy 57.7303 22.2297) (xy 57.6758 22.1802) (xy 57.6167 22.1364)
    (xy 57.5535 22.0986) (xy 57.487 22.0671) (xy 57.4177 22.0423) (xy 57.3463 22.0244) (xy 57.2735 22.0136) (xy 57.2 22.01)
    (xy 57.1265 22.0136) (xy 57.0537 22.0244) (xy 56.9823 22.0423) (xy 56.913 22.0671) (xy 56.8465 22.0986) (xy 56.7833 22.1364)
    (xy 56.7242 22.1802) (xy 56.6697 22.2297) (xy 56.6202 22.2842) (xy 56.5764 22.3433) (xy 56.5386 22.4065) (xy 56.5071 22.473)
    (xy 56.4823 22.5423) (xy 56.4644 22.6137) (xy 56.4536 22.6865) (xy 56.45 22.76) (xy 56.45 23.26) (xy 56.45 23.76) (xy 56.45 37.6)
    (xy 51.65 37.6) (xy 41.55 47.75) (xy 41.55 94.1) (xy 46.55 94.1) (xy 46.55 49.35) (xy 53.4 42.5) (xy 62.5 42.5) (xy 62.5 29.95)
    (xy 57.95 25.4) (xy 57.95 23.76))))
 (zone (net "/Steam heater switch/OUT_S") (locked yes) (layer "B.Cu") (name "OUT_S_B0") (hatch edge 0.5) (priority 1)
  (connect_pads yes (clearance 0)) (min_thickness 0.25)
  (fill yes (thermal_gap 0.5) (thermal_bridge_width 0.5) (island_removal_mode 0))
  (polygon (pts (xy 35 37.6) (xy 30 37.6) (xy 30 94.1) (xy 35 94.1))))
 (segment (start 60.640000 58.200000) (end 60.640000 54.955000) (width 0.2) (layer "F.Cu") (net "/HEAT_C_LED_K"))
 (segment (start 63.180000 58.200000) (end 63.180000 61.445000) (width 0.2) (layer "F.Cu") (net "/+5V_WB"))
 (segment (start 63.180000 58.200000) (end 61.630000 56.650000) (width 0.2) (layer "B.Cu") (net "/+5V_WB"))
 (segment (start 61.630000 56.650000) (end 58.100000 56.650000) (width 0.2) (layer "B.Cu") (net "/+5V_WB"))
 (via (at 58.1 56.65) (size 0.7) (drill 0.3) (layers "F.Cu" "B.Cu") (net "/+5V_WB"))
 (segment (start 58.100000 56.650000) (end 58.100000 54.955000) (width 0.2) (layer "F.Cu") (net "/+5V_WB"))
 (segment (start 58.100000 58.200000) (end 60.640000 60.740000) (width 0.2) (layer "F.Cu") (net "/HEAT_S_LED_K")))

